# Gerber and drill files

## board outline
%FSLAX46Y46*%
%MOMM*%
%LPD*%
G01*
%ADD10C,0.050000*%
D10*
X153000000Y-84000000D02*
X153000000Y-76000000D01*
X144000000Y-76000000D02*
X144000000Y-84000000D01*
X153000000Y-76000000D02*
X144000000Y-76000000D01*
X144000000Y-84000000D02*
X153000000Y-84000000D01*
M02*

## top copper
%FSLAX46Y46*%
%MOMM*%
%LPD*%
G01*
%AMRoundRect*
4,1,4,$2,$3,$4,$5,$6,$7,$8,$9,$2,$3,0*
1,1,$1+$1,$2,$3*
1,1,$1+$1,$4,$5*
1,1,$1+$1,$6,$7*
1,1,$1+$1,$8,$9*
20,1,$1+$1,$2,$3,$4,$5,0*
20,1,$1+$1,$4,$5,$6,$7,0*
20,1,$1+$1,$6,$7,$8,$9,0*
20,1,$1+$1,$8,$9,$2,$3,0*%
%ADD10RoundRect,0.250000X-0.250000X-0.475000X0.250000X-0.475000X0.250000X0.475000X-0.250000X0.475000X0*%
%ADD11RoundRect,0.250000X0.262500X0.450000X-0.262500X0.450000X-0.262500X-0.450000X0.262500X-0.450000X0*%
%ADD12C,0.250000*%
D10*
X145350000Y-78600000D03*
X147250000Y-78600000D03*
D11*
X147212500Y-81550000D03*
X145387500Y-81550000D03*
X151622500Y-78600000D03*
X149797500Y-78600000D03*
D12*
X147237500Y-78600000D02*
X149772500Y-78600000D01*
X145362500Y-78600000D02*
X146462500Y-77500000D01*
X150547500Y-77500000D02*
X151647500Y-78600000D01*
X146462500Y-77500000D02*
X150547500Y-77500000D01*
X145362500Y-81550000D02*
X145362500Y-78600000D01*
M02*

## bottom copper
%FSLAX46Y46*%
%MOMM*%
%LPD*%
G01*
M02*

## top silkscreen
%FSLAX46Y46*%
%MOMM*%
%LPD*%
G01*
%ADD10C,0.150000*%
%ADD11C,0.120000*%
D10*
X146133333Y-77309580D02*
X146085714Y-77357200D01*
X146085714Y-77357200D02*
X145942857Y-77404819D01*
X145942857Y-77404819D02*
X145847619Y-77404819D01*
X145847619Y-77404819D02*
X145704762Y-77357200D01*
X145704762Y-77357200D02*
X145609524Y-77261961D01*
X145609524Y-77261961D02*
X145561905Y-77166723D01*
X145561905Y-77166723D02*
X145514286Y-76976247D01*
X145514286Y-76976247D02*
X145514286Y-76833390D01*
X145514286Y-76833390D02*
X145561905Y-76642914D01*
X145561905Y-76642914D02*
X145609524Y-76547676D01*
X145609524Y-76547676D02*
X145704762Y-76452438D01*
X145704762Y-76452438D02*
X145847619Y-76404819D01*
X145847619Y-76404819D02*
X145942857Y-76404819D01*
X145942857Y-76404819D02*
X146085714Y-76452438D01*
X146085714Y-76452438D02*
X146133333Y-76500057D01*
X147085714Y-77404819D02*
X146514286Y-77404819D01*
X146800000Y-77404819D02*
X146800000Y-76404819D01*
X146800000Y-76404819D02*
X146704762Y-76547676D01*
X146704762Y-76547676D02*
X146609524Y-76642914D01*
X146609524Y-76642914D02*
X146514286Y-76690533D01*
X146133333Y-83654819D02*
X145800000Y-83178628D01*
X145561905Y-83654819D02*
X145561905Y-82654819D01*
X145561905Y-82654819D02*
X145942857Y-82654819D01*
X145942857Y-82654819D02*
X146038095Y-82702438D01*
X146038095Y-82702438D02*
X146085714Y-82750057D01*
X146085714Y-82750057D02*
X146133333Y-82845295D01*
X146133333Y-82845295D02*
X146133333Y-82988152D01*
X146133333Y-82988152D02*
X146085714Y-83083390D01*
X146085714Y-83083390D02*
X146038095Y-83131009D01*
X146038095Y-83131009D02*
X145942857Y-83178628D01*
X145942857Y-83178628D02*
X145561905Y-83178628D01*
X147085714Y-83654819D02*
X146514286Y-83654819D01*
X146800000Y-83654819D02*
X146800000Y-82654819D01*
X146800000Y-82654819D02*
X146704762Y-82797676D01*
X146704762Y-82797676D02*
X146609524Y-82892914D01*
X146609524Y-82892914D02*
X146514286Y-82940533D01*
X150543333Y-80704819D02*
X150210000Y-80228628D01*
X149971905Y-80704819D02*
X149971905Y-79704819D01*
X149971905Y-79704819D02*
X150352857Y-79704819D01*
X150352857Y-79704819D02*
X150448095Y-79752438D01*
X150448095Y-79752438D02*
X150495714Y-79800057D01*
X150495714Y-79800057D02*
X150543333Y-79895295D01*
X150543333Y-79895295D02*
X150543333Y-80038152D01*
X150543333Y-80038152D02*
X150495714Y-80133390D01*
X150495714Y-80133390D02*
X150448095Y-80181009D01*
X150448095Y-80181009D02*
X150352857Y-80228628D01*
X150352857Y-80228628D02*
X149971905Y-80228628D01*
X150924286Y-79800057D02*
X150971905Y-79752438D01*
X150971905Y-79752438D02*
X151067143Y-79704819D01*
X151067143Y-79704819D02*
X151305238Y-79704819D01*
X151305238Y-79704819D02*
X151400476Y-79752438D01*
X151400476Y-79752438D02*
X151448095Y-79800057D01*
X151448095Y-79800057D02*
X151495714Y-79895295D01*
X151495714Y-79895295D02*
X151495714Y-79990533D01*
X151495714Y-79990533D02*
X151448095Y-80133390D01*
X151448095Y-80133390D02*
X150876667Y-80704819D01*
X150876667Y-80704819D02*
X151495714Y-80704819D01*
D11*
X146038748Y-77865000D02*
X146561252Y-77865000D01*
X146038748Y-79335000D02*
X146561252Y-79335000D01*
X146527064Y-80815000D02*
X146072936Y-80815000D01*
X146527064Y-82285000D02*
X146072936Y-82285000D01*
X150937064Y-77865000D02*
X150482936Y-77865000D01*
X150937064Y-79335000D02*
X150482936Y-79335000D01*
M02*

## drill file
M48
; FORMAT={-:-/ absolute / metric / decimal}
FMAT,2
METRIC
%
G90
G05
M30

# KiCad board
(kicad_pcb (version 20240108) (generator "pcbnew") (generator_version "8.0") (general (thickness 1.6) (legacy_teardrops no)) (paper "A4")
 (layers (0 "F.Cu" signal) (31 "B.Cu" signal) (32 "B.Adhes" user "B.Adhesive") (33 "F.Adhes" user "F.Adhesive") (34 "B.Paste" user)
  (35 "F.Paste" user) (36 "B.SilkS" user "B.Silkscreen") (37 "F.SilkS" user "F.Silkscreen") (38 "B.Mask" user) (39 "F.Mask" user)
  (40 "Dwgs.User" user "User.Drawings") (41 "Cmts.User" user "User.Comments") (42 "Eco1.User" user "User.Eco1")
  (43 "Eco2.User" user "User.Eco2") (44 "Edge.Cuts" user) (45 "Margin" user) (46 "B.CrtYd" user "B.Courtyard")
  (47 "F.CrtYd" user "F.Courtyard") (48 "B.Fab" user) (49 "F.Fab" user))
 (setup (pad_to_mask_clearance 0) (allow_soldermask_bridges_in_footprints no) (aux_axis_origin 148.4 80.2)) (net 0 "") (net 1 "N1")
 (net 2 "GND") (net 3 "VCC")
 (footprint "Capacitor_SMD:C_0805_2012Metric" (layer "F.Cu") (at 146.3 78.6)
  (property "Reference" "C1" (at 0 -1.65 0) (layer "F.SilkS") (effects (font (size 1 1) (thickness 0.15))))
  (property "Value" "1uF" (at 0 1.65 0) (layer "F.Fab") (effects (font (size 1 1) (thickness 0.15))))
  (fp_line (start -0.261252 -0.735) (end 0.261252 -0.735) (stroke (width 0.12) (type solid)) (layer "F.SilkS"))
  (fp_line (start -0.261252 0.735) (end 0.261252 0.735) (stroke (width 0.12) (type solid)) (layer "F.SilkS"))
  (pad "1" smd roundrect (at -0.95 0) (size 1 1.45) (layers "F.Cu" "F.Paste" "F.Mask") (roundrect_rratio 0.25) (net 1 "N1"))
  (pad "2" smd roundrect (at 0.95 0) (size 1 1.45) (layers "F.Cu" "F.Paste" "F.Mask") (roundrect_rratio 0.25) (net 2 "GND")))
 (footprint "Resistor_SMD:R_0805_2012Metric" (layer "F.Cu") (at 146.3 81.55 180)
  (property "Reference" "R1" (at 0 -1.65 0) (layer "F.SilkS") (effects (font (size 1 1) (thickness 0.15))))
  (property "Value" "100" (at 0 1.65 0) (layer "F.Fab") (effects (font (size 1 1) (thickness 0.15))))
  (fp_line (start -0.227064 0.735) (end 0.227064 0.735) (stroke (width 0.12) (type solid)) (layer "F.SilkS"))
  (fp_line (start -0.227064 -0.735) (end 0.227064 -0.735) (stroke (width 0.12) (type solid)) (layer "F.SilkS"))
  (pad "1" smd roundrect (at -0.9125 0 180) (size 1.025 1.4) (layers "F.Cu" "F.Paste" "F.Mask") (roundrect_rratio 0.243902) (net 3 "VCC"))
  (pad "2" smd roundrect (at 0.9125 0 180) (size 1.025 1.4) (layers "F.Cu" "F.Paste" "F.Mask") (roundrect_rratio 0.243902) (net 1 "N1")))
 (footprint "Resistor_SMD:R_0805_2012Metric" (layer "F.Cu") (at 150.71 78.6 180)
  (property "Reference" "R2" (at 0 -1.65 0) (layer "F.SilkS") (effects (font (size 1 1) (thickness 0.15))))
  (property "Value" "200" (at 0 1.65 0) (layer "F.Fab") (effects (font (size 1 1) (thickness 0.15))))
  (fp_line (start -0.227064 0.735) (end 0.227064 0.735) (stroke (width 0.12) (type solid)) (layer "F.SilkS"))
  (fp_line (start -0.227064 -0.735) (end 0.227064 -0.735) (stroke (width 0.12) (type solid)) (layer "F.SilkS"))
  (pad "1" smd roundrect (at -0.9125 0 180) (size 1.025 1.4) (layers "F.Cu" "F.Paste" "F.Mask") (roundrect_rratio 0.243902) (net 1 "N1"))
  (pad "2" smd roundrect (at 0.9125 0 180) (size 1.025 1.4) (layers "F.Cu" "F.Paste" "F.Mask") (roundrect_rratio 0.243902) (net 2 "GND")))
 (gr_line (start 153 84) (end 153 76) (stroke (width 0.05) (type solid)) (layer "Edge.Cuts"))
 (gr_line (start 144 76) (end 144 84) (stroke (width 0.05) (type solid)) (layer "Edge.Cuts"))
 (gr_line (start 153 76) (end 144 76) (stroke (width 0.05) (type solid)) (layer "Edge.Cuts"))
 (gr_line (start 144 84) (end 153 84) (stroke (width 0.05) (type solid)) (layer "Edge.Cuts"))
 (segment (start 147.2375 78.6) (end 149.7725 78.6) (width 0.25) (layer "F.Cu") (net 2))
 (segment (start 145.3625 78.6) (end 146.4625 77.5) (width 0.25) (layer "F.Cu") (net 1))
 (segment (start 150.5475 77.5) (end 151.6475 78.6) (width 0.25) (layer "F.Cu") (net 1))
 (segment (start 146.4625 77.5) (end 150.5475 77.5) (width 0.25) (layer "F.Cu") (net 1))
 (segment (start 145.3625 81.55) (end 145.3625 78.6) (width 0.25) (layer "F.Cu") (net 1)))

